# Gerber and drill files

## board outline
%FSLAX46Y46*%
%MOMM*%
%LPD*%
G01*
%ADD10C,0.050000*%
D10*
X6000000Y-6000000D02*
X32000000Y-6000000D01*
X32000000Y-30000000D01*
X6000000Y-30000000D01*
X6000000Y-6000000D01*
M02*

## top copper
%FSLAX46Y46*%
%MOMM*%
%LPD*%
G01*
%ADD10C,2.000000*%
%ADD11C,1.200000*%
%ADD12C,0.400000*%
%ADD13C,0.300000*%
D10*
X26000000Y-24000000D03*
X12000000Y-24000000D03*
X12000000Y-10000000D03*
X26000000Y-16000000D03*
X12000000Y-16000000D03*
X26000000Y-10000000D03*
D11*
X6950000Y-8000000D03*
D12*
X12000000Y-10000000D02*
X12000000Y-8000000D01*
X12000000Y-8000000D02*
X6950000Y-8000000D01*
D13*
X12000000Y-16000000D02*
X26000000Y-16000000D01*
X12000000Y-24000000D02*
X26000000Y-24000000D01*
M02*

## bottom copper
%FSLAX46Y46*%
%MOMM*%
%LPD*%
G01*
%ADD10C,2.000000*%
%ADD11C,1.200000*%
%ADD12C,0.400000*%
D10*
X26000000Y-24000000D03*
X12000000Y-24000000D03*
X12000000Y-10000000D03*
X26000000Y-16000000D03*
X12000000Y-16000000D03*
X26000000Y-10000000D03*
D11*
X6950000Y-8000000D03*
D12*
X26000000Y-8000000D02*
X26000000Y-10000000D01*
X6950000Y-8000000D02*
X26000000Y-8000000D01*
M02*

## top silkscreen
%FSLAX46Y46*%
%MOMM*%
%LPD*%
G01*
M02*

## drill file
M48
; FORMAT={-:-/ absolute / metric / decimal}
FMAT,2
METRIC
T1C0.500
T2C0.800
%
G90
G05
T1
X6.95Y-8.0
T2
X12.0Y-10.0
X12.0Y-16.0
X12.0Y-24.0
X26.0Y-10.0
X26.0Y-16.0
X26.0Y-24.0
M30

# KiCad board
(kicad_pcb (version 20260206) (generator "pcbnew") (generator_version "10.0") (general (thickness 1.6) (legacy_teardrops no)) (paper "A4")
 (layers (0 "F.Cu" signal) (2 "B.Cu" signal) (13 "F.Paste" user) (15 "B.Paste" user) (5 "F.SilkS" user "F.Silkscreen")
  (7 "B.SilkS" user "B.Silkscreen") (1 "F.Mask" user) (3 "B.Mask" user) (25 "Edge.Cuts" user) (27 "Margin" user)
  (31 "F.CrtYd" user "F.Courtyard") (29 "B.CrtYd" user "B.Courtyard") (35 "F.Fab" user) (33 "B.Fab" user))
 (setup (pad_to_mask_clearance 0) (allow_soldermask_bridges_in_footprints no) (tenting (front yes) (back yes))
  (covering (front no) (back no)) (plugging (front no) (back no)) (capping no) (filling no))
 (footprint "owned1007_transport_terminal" (layer "F.Cu") (at 26 24)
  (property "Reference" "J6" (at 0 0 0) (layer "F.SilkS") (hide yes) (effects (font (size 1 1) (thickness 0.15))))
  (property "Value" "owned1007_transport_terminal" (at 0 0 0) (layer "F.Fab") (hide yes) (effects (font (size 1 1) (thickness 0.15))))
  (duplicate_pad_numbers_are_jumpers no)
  (pad "1" thru_hole circle (at 0 0) (size 2 2) (drill 0.8) (layers "*.Cu" "*.Mask") (remove_unused_layers no) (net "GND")))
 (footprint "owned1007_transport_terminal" (layer "F.Cu") (at 12 24)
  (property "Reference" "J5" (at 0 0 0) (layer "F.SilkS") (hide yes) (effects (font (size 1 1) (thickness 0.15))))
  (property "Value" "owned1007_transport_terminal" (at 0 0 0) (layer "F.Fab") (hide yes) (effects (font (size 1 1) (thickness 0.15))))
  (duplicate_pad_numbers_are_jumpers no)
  (pad "1" thru_hole circle (at 0 0) (size 2 2) (drill 0.8) (layers "*.Cu" "*.Mask") (remove_unused_layers no) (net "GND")))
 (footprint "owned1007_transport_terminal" (layer "F.Cu") (at 12 10)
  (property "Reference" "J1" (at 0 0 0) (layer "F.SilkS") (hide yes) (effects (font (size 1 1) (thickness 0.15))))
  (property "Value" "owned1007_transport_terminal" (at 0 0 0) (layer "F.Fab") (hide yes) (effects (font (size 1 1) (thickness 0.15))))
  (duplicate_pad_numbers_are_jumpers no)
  (pad "1" thru_hole circle (at 0 0) (size 2 2) (drill 0.8) (layers "*.Cu" "*.Mask") (remove_unused_layers no) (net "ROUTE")))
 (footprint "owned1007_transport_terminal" (layer "F.Cu") (at 26 16)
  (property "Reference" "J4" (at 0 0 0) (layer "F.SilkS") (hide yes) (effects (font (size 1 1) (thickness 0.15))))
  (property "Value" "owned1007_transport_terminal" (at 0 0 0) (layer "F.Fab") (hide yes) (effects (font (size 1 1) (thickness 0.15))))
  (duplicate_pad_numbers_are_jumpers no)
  (pad "1" thru_hole circle (at 0 0) (size 2 2) (drill 0.8) (layers "*.Cu" "*.Mask") (remove_unused_layers no) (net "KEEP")))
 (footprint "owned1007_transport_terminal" (layer "F.Cu") (at 12 16)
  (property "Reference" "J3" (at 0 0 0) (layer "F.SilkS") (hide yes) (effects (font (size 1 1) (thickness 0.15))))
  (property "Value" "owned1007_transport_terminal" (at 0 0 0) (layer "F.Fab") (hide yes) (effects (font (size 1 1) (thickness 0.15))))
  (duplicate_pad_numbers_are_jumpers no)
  (pad "1" thru_hole circle (at 0 0) (size 2 2) (drill 0.8) (layers "*.Cu" "*.Mask") (remove_unused_layers no) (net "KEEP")))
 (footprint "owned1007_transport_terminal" (layer "F.Cu") (at 26 10)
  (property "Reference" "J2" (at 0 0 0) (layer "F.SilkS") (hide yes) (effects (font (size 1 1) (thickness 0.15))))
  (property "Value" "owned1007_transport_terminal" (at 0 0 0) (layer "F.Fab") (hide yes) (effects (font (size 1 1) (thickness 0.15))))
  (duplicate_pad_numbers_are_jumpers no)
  (pad "1" thru_hole circle (at 0 0) (size 2 2) (drill 0.8) (layers "*.Cu" "*.Mask") (remove_unused_layers no) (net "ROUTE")))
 (gr_rect (start 6 6) (end 32 30) (stroke (width 0.05) (type default)) (fill no) (layer "Edge.Cuts"))
 (segment (start 12 10) (end 12 8) (width 0.4) (layer "F.Cu") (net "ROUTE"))
 (segment (start 12 8) (end 6.95 8) (width 0.4) (layer "F.Cu") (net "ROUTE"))
 (via (at 6.95 8) (size 1.2) (drill 0.5) (layers "F.Cu" "B.Cu") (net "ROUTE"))
 (segment (start 26 8) (end 26 10) (width 0.4) (layer "B.Cu") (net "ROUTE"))
 (segment (start 6.95 8) (end 26 8) (width 0.4) (layer "B.Cu") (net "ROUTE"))
 (segment (start 12 16) (end 26 16) (width 0.3) (locked yes) (layer "F.Cu") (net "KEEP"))
 (segment (start 12 24) (end 26 24) (width 0.3) (layer "F.Cu") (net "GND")))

